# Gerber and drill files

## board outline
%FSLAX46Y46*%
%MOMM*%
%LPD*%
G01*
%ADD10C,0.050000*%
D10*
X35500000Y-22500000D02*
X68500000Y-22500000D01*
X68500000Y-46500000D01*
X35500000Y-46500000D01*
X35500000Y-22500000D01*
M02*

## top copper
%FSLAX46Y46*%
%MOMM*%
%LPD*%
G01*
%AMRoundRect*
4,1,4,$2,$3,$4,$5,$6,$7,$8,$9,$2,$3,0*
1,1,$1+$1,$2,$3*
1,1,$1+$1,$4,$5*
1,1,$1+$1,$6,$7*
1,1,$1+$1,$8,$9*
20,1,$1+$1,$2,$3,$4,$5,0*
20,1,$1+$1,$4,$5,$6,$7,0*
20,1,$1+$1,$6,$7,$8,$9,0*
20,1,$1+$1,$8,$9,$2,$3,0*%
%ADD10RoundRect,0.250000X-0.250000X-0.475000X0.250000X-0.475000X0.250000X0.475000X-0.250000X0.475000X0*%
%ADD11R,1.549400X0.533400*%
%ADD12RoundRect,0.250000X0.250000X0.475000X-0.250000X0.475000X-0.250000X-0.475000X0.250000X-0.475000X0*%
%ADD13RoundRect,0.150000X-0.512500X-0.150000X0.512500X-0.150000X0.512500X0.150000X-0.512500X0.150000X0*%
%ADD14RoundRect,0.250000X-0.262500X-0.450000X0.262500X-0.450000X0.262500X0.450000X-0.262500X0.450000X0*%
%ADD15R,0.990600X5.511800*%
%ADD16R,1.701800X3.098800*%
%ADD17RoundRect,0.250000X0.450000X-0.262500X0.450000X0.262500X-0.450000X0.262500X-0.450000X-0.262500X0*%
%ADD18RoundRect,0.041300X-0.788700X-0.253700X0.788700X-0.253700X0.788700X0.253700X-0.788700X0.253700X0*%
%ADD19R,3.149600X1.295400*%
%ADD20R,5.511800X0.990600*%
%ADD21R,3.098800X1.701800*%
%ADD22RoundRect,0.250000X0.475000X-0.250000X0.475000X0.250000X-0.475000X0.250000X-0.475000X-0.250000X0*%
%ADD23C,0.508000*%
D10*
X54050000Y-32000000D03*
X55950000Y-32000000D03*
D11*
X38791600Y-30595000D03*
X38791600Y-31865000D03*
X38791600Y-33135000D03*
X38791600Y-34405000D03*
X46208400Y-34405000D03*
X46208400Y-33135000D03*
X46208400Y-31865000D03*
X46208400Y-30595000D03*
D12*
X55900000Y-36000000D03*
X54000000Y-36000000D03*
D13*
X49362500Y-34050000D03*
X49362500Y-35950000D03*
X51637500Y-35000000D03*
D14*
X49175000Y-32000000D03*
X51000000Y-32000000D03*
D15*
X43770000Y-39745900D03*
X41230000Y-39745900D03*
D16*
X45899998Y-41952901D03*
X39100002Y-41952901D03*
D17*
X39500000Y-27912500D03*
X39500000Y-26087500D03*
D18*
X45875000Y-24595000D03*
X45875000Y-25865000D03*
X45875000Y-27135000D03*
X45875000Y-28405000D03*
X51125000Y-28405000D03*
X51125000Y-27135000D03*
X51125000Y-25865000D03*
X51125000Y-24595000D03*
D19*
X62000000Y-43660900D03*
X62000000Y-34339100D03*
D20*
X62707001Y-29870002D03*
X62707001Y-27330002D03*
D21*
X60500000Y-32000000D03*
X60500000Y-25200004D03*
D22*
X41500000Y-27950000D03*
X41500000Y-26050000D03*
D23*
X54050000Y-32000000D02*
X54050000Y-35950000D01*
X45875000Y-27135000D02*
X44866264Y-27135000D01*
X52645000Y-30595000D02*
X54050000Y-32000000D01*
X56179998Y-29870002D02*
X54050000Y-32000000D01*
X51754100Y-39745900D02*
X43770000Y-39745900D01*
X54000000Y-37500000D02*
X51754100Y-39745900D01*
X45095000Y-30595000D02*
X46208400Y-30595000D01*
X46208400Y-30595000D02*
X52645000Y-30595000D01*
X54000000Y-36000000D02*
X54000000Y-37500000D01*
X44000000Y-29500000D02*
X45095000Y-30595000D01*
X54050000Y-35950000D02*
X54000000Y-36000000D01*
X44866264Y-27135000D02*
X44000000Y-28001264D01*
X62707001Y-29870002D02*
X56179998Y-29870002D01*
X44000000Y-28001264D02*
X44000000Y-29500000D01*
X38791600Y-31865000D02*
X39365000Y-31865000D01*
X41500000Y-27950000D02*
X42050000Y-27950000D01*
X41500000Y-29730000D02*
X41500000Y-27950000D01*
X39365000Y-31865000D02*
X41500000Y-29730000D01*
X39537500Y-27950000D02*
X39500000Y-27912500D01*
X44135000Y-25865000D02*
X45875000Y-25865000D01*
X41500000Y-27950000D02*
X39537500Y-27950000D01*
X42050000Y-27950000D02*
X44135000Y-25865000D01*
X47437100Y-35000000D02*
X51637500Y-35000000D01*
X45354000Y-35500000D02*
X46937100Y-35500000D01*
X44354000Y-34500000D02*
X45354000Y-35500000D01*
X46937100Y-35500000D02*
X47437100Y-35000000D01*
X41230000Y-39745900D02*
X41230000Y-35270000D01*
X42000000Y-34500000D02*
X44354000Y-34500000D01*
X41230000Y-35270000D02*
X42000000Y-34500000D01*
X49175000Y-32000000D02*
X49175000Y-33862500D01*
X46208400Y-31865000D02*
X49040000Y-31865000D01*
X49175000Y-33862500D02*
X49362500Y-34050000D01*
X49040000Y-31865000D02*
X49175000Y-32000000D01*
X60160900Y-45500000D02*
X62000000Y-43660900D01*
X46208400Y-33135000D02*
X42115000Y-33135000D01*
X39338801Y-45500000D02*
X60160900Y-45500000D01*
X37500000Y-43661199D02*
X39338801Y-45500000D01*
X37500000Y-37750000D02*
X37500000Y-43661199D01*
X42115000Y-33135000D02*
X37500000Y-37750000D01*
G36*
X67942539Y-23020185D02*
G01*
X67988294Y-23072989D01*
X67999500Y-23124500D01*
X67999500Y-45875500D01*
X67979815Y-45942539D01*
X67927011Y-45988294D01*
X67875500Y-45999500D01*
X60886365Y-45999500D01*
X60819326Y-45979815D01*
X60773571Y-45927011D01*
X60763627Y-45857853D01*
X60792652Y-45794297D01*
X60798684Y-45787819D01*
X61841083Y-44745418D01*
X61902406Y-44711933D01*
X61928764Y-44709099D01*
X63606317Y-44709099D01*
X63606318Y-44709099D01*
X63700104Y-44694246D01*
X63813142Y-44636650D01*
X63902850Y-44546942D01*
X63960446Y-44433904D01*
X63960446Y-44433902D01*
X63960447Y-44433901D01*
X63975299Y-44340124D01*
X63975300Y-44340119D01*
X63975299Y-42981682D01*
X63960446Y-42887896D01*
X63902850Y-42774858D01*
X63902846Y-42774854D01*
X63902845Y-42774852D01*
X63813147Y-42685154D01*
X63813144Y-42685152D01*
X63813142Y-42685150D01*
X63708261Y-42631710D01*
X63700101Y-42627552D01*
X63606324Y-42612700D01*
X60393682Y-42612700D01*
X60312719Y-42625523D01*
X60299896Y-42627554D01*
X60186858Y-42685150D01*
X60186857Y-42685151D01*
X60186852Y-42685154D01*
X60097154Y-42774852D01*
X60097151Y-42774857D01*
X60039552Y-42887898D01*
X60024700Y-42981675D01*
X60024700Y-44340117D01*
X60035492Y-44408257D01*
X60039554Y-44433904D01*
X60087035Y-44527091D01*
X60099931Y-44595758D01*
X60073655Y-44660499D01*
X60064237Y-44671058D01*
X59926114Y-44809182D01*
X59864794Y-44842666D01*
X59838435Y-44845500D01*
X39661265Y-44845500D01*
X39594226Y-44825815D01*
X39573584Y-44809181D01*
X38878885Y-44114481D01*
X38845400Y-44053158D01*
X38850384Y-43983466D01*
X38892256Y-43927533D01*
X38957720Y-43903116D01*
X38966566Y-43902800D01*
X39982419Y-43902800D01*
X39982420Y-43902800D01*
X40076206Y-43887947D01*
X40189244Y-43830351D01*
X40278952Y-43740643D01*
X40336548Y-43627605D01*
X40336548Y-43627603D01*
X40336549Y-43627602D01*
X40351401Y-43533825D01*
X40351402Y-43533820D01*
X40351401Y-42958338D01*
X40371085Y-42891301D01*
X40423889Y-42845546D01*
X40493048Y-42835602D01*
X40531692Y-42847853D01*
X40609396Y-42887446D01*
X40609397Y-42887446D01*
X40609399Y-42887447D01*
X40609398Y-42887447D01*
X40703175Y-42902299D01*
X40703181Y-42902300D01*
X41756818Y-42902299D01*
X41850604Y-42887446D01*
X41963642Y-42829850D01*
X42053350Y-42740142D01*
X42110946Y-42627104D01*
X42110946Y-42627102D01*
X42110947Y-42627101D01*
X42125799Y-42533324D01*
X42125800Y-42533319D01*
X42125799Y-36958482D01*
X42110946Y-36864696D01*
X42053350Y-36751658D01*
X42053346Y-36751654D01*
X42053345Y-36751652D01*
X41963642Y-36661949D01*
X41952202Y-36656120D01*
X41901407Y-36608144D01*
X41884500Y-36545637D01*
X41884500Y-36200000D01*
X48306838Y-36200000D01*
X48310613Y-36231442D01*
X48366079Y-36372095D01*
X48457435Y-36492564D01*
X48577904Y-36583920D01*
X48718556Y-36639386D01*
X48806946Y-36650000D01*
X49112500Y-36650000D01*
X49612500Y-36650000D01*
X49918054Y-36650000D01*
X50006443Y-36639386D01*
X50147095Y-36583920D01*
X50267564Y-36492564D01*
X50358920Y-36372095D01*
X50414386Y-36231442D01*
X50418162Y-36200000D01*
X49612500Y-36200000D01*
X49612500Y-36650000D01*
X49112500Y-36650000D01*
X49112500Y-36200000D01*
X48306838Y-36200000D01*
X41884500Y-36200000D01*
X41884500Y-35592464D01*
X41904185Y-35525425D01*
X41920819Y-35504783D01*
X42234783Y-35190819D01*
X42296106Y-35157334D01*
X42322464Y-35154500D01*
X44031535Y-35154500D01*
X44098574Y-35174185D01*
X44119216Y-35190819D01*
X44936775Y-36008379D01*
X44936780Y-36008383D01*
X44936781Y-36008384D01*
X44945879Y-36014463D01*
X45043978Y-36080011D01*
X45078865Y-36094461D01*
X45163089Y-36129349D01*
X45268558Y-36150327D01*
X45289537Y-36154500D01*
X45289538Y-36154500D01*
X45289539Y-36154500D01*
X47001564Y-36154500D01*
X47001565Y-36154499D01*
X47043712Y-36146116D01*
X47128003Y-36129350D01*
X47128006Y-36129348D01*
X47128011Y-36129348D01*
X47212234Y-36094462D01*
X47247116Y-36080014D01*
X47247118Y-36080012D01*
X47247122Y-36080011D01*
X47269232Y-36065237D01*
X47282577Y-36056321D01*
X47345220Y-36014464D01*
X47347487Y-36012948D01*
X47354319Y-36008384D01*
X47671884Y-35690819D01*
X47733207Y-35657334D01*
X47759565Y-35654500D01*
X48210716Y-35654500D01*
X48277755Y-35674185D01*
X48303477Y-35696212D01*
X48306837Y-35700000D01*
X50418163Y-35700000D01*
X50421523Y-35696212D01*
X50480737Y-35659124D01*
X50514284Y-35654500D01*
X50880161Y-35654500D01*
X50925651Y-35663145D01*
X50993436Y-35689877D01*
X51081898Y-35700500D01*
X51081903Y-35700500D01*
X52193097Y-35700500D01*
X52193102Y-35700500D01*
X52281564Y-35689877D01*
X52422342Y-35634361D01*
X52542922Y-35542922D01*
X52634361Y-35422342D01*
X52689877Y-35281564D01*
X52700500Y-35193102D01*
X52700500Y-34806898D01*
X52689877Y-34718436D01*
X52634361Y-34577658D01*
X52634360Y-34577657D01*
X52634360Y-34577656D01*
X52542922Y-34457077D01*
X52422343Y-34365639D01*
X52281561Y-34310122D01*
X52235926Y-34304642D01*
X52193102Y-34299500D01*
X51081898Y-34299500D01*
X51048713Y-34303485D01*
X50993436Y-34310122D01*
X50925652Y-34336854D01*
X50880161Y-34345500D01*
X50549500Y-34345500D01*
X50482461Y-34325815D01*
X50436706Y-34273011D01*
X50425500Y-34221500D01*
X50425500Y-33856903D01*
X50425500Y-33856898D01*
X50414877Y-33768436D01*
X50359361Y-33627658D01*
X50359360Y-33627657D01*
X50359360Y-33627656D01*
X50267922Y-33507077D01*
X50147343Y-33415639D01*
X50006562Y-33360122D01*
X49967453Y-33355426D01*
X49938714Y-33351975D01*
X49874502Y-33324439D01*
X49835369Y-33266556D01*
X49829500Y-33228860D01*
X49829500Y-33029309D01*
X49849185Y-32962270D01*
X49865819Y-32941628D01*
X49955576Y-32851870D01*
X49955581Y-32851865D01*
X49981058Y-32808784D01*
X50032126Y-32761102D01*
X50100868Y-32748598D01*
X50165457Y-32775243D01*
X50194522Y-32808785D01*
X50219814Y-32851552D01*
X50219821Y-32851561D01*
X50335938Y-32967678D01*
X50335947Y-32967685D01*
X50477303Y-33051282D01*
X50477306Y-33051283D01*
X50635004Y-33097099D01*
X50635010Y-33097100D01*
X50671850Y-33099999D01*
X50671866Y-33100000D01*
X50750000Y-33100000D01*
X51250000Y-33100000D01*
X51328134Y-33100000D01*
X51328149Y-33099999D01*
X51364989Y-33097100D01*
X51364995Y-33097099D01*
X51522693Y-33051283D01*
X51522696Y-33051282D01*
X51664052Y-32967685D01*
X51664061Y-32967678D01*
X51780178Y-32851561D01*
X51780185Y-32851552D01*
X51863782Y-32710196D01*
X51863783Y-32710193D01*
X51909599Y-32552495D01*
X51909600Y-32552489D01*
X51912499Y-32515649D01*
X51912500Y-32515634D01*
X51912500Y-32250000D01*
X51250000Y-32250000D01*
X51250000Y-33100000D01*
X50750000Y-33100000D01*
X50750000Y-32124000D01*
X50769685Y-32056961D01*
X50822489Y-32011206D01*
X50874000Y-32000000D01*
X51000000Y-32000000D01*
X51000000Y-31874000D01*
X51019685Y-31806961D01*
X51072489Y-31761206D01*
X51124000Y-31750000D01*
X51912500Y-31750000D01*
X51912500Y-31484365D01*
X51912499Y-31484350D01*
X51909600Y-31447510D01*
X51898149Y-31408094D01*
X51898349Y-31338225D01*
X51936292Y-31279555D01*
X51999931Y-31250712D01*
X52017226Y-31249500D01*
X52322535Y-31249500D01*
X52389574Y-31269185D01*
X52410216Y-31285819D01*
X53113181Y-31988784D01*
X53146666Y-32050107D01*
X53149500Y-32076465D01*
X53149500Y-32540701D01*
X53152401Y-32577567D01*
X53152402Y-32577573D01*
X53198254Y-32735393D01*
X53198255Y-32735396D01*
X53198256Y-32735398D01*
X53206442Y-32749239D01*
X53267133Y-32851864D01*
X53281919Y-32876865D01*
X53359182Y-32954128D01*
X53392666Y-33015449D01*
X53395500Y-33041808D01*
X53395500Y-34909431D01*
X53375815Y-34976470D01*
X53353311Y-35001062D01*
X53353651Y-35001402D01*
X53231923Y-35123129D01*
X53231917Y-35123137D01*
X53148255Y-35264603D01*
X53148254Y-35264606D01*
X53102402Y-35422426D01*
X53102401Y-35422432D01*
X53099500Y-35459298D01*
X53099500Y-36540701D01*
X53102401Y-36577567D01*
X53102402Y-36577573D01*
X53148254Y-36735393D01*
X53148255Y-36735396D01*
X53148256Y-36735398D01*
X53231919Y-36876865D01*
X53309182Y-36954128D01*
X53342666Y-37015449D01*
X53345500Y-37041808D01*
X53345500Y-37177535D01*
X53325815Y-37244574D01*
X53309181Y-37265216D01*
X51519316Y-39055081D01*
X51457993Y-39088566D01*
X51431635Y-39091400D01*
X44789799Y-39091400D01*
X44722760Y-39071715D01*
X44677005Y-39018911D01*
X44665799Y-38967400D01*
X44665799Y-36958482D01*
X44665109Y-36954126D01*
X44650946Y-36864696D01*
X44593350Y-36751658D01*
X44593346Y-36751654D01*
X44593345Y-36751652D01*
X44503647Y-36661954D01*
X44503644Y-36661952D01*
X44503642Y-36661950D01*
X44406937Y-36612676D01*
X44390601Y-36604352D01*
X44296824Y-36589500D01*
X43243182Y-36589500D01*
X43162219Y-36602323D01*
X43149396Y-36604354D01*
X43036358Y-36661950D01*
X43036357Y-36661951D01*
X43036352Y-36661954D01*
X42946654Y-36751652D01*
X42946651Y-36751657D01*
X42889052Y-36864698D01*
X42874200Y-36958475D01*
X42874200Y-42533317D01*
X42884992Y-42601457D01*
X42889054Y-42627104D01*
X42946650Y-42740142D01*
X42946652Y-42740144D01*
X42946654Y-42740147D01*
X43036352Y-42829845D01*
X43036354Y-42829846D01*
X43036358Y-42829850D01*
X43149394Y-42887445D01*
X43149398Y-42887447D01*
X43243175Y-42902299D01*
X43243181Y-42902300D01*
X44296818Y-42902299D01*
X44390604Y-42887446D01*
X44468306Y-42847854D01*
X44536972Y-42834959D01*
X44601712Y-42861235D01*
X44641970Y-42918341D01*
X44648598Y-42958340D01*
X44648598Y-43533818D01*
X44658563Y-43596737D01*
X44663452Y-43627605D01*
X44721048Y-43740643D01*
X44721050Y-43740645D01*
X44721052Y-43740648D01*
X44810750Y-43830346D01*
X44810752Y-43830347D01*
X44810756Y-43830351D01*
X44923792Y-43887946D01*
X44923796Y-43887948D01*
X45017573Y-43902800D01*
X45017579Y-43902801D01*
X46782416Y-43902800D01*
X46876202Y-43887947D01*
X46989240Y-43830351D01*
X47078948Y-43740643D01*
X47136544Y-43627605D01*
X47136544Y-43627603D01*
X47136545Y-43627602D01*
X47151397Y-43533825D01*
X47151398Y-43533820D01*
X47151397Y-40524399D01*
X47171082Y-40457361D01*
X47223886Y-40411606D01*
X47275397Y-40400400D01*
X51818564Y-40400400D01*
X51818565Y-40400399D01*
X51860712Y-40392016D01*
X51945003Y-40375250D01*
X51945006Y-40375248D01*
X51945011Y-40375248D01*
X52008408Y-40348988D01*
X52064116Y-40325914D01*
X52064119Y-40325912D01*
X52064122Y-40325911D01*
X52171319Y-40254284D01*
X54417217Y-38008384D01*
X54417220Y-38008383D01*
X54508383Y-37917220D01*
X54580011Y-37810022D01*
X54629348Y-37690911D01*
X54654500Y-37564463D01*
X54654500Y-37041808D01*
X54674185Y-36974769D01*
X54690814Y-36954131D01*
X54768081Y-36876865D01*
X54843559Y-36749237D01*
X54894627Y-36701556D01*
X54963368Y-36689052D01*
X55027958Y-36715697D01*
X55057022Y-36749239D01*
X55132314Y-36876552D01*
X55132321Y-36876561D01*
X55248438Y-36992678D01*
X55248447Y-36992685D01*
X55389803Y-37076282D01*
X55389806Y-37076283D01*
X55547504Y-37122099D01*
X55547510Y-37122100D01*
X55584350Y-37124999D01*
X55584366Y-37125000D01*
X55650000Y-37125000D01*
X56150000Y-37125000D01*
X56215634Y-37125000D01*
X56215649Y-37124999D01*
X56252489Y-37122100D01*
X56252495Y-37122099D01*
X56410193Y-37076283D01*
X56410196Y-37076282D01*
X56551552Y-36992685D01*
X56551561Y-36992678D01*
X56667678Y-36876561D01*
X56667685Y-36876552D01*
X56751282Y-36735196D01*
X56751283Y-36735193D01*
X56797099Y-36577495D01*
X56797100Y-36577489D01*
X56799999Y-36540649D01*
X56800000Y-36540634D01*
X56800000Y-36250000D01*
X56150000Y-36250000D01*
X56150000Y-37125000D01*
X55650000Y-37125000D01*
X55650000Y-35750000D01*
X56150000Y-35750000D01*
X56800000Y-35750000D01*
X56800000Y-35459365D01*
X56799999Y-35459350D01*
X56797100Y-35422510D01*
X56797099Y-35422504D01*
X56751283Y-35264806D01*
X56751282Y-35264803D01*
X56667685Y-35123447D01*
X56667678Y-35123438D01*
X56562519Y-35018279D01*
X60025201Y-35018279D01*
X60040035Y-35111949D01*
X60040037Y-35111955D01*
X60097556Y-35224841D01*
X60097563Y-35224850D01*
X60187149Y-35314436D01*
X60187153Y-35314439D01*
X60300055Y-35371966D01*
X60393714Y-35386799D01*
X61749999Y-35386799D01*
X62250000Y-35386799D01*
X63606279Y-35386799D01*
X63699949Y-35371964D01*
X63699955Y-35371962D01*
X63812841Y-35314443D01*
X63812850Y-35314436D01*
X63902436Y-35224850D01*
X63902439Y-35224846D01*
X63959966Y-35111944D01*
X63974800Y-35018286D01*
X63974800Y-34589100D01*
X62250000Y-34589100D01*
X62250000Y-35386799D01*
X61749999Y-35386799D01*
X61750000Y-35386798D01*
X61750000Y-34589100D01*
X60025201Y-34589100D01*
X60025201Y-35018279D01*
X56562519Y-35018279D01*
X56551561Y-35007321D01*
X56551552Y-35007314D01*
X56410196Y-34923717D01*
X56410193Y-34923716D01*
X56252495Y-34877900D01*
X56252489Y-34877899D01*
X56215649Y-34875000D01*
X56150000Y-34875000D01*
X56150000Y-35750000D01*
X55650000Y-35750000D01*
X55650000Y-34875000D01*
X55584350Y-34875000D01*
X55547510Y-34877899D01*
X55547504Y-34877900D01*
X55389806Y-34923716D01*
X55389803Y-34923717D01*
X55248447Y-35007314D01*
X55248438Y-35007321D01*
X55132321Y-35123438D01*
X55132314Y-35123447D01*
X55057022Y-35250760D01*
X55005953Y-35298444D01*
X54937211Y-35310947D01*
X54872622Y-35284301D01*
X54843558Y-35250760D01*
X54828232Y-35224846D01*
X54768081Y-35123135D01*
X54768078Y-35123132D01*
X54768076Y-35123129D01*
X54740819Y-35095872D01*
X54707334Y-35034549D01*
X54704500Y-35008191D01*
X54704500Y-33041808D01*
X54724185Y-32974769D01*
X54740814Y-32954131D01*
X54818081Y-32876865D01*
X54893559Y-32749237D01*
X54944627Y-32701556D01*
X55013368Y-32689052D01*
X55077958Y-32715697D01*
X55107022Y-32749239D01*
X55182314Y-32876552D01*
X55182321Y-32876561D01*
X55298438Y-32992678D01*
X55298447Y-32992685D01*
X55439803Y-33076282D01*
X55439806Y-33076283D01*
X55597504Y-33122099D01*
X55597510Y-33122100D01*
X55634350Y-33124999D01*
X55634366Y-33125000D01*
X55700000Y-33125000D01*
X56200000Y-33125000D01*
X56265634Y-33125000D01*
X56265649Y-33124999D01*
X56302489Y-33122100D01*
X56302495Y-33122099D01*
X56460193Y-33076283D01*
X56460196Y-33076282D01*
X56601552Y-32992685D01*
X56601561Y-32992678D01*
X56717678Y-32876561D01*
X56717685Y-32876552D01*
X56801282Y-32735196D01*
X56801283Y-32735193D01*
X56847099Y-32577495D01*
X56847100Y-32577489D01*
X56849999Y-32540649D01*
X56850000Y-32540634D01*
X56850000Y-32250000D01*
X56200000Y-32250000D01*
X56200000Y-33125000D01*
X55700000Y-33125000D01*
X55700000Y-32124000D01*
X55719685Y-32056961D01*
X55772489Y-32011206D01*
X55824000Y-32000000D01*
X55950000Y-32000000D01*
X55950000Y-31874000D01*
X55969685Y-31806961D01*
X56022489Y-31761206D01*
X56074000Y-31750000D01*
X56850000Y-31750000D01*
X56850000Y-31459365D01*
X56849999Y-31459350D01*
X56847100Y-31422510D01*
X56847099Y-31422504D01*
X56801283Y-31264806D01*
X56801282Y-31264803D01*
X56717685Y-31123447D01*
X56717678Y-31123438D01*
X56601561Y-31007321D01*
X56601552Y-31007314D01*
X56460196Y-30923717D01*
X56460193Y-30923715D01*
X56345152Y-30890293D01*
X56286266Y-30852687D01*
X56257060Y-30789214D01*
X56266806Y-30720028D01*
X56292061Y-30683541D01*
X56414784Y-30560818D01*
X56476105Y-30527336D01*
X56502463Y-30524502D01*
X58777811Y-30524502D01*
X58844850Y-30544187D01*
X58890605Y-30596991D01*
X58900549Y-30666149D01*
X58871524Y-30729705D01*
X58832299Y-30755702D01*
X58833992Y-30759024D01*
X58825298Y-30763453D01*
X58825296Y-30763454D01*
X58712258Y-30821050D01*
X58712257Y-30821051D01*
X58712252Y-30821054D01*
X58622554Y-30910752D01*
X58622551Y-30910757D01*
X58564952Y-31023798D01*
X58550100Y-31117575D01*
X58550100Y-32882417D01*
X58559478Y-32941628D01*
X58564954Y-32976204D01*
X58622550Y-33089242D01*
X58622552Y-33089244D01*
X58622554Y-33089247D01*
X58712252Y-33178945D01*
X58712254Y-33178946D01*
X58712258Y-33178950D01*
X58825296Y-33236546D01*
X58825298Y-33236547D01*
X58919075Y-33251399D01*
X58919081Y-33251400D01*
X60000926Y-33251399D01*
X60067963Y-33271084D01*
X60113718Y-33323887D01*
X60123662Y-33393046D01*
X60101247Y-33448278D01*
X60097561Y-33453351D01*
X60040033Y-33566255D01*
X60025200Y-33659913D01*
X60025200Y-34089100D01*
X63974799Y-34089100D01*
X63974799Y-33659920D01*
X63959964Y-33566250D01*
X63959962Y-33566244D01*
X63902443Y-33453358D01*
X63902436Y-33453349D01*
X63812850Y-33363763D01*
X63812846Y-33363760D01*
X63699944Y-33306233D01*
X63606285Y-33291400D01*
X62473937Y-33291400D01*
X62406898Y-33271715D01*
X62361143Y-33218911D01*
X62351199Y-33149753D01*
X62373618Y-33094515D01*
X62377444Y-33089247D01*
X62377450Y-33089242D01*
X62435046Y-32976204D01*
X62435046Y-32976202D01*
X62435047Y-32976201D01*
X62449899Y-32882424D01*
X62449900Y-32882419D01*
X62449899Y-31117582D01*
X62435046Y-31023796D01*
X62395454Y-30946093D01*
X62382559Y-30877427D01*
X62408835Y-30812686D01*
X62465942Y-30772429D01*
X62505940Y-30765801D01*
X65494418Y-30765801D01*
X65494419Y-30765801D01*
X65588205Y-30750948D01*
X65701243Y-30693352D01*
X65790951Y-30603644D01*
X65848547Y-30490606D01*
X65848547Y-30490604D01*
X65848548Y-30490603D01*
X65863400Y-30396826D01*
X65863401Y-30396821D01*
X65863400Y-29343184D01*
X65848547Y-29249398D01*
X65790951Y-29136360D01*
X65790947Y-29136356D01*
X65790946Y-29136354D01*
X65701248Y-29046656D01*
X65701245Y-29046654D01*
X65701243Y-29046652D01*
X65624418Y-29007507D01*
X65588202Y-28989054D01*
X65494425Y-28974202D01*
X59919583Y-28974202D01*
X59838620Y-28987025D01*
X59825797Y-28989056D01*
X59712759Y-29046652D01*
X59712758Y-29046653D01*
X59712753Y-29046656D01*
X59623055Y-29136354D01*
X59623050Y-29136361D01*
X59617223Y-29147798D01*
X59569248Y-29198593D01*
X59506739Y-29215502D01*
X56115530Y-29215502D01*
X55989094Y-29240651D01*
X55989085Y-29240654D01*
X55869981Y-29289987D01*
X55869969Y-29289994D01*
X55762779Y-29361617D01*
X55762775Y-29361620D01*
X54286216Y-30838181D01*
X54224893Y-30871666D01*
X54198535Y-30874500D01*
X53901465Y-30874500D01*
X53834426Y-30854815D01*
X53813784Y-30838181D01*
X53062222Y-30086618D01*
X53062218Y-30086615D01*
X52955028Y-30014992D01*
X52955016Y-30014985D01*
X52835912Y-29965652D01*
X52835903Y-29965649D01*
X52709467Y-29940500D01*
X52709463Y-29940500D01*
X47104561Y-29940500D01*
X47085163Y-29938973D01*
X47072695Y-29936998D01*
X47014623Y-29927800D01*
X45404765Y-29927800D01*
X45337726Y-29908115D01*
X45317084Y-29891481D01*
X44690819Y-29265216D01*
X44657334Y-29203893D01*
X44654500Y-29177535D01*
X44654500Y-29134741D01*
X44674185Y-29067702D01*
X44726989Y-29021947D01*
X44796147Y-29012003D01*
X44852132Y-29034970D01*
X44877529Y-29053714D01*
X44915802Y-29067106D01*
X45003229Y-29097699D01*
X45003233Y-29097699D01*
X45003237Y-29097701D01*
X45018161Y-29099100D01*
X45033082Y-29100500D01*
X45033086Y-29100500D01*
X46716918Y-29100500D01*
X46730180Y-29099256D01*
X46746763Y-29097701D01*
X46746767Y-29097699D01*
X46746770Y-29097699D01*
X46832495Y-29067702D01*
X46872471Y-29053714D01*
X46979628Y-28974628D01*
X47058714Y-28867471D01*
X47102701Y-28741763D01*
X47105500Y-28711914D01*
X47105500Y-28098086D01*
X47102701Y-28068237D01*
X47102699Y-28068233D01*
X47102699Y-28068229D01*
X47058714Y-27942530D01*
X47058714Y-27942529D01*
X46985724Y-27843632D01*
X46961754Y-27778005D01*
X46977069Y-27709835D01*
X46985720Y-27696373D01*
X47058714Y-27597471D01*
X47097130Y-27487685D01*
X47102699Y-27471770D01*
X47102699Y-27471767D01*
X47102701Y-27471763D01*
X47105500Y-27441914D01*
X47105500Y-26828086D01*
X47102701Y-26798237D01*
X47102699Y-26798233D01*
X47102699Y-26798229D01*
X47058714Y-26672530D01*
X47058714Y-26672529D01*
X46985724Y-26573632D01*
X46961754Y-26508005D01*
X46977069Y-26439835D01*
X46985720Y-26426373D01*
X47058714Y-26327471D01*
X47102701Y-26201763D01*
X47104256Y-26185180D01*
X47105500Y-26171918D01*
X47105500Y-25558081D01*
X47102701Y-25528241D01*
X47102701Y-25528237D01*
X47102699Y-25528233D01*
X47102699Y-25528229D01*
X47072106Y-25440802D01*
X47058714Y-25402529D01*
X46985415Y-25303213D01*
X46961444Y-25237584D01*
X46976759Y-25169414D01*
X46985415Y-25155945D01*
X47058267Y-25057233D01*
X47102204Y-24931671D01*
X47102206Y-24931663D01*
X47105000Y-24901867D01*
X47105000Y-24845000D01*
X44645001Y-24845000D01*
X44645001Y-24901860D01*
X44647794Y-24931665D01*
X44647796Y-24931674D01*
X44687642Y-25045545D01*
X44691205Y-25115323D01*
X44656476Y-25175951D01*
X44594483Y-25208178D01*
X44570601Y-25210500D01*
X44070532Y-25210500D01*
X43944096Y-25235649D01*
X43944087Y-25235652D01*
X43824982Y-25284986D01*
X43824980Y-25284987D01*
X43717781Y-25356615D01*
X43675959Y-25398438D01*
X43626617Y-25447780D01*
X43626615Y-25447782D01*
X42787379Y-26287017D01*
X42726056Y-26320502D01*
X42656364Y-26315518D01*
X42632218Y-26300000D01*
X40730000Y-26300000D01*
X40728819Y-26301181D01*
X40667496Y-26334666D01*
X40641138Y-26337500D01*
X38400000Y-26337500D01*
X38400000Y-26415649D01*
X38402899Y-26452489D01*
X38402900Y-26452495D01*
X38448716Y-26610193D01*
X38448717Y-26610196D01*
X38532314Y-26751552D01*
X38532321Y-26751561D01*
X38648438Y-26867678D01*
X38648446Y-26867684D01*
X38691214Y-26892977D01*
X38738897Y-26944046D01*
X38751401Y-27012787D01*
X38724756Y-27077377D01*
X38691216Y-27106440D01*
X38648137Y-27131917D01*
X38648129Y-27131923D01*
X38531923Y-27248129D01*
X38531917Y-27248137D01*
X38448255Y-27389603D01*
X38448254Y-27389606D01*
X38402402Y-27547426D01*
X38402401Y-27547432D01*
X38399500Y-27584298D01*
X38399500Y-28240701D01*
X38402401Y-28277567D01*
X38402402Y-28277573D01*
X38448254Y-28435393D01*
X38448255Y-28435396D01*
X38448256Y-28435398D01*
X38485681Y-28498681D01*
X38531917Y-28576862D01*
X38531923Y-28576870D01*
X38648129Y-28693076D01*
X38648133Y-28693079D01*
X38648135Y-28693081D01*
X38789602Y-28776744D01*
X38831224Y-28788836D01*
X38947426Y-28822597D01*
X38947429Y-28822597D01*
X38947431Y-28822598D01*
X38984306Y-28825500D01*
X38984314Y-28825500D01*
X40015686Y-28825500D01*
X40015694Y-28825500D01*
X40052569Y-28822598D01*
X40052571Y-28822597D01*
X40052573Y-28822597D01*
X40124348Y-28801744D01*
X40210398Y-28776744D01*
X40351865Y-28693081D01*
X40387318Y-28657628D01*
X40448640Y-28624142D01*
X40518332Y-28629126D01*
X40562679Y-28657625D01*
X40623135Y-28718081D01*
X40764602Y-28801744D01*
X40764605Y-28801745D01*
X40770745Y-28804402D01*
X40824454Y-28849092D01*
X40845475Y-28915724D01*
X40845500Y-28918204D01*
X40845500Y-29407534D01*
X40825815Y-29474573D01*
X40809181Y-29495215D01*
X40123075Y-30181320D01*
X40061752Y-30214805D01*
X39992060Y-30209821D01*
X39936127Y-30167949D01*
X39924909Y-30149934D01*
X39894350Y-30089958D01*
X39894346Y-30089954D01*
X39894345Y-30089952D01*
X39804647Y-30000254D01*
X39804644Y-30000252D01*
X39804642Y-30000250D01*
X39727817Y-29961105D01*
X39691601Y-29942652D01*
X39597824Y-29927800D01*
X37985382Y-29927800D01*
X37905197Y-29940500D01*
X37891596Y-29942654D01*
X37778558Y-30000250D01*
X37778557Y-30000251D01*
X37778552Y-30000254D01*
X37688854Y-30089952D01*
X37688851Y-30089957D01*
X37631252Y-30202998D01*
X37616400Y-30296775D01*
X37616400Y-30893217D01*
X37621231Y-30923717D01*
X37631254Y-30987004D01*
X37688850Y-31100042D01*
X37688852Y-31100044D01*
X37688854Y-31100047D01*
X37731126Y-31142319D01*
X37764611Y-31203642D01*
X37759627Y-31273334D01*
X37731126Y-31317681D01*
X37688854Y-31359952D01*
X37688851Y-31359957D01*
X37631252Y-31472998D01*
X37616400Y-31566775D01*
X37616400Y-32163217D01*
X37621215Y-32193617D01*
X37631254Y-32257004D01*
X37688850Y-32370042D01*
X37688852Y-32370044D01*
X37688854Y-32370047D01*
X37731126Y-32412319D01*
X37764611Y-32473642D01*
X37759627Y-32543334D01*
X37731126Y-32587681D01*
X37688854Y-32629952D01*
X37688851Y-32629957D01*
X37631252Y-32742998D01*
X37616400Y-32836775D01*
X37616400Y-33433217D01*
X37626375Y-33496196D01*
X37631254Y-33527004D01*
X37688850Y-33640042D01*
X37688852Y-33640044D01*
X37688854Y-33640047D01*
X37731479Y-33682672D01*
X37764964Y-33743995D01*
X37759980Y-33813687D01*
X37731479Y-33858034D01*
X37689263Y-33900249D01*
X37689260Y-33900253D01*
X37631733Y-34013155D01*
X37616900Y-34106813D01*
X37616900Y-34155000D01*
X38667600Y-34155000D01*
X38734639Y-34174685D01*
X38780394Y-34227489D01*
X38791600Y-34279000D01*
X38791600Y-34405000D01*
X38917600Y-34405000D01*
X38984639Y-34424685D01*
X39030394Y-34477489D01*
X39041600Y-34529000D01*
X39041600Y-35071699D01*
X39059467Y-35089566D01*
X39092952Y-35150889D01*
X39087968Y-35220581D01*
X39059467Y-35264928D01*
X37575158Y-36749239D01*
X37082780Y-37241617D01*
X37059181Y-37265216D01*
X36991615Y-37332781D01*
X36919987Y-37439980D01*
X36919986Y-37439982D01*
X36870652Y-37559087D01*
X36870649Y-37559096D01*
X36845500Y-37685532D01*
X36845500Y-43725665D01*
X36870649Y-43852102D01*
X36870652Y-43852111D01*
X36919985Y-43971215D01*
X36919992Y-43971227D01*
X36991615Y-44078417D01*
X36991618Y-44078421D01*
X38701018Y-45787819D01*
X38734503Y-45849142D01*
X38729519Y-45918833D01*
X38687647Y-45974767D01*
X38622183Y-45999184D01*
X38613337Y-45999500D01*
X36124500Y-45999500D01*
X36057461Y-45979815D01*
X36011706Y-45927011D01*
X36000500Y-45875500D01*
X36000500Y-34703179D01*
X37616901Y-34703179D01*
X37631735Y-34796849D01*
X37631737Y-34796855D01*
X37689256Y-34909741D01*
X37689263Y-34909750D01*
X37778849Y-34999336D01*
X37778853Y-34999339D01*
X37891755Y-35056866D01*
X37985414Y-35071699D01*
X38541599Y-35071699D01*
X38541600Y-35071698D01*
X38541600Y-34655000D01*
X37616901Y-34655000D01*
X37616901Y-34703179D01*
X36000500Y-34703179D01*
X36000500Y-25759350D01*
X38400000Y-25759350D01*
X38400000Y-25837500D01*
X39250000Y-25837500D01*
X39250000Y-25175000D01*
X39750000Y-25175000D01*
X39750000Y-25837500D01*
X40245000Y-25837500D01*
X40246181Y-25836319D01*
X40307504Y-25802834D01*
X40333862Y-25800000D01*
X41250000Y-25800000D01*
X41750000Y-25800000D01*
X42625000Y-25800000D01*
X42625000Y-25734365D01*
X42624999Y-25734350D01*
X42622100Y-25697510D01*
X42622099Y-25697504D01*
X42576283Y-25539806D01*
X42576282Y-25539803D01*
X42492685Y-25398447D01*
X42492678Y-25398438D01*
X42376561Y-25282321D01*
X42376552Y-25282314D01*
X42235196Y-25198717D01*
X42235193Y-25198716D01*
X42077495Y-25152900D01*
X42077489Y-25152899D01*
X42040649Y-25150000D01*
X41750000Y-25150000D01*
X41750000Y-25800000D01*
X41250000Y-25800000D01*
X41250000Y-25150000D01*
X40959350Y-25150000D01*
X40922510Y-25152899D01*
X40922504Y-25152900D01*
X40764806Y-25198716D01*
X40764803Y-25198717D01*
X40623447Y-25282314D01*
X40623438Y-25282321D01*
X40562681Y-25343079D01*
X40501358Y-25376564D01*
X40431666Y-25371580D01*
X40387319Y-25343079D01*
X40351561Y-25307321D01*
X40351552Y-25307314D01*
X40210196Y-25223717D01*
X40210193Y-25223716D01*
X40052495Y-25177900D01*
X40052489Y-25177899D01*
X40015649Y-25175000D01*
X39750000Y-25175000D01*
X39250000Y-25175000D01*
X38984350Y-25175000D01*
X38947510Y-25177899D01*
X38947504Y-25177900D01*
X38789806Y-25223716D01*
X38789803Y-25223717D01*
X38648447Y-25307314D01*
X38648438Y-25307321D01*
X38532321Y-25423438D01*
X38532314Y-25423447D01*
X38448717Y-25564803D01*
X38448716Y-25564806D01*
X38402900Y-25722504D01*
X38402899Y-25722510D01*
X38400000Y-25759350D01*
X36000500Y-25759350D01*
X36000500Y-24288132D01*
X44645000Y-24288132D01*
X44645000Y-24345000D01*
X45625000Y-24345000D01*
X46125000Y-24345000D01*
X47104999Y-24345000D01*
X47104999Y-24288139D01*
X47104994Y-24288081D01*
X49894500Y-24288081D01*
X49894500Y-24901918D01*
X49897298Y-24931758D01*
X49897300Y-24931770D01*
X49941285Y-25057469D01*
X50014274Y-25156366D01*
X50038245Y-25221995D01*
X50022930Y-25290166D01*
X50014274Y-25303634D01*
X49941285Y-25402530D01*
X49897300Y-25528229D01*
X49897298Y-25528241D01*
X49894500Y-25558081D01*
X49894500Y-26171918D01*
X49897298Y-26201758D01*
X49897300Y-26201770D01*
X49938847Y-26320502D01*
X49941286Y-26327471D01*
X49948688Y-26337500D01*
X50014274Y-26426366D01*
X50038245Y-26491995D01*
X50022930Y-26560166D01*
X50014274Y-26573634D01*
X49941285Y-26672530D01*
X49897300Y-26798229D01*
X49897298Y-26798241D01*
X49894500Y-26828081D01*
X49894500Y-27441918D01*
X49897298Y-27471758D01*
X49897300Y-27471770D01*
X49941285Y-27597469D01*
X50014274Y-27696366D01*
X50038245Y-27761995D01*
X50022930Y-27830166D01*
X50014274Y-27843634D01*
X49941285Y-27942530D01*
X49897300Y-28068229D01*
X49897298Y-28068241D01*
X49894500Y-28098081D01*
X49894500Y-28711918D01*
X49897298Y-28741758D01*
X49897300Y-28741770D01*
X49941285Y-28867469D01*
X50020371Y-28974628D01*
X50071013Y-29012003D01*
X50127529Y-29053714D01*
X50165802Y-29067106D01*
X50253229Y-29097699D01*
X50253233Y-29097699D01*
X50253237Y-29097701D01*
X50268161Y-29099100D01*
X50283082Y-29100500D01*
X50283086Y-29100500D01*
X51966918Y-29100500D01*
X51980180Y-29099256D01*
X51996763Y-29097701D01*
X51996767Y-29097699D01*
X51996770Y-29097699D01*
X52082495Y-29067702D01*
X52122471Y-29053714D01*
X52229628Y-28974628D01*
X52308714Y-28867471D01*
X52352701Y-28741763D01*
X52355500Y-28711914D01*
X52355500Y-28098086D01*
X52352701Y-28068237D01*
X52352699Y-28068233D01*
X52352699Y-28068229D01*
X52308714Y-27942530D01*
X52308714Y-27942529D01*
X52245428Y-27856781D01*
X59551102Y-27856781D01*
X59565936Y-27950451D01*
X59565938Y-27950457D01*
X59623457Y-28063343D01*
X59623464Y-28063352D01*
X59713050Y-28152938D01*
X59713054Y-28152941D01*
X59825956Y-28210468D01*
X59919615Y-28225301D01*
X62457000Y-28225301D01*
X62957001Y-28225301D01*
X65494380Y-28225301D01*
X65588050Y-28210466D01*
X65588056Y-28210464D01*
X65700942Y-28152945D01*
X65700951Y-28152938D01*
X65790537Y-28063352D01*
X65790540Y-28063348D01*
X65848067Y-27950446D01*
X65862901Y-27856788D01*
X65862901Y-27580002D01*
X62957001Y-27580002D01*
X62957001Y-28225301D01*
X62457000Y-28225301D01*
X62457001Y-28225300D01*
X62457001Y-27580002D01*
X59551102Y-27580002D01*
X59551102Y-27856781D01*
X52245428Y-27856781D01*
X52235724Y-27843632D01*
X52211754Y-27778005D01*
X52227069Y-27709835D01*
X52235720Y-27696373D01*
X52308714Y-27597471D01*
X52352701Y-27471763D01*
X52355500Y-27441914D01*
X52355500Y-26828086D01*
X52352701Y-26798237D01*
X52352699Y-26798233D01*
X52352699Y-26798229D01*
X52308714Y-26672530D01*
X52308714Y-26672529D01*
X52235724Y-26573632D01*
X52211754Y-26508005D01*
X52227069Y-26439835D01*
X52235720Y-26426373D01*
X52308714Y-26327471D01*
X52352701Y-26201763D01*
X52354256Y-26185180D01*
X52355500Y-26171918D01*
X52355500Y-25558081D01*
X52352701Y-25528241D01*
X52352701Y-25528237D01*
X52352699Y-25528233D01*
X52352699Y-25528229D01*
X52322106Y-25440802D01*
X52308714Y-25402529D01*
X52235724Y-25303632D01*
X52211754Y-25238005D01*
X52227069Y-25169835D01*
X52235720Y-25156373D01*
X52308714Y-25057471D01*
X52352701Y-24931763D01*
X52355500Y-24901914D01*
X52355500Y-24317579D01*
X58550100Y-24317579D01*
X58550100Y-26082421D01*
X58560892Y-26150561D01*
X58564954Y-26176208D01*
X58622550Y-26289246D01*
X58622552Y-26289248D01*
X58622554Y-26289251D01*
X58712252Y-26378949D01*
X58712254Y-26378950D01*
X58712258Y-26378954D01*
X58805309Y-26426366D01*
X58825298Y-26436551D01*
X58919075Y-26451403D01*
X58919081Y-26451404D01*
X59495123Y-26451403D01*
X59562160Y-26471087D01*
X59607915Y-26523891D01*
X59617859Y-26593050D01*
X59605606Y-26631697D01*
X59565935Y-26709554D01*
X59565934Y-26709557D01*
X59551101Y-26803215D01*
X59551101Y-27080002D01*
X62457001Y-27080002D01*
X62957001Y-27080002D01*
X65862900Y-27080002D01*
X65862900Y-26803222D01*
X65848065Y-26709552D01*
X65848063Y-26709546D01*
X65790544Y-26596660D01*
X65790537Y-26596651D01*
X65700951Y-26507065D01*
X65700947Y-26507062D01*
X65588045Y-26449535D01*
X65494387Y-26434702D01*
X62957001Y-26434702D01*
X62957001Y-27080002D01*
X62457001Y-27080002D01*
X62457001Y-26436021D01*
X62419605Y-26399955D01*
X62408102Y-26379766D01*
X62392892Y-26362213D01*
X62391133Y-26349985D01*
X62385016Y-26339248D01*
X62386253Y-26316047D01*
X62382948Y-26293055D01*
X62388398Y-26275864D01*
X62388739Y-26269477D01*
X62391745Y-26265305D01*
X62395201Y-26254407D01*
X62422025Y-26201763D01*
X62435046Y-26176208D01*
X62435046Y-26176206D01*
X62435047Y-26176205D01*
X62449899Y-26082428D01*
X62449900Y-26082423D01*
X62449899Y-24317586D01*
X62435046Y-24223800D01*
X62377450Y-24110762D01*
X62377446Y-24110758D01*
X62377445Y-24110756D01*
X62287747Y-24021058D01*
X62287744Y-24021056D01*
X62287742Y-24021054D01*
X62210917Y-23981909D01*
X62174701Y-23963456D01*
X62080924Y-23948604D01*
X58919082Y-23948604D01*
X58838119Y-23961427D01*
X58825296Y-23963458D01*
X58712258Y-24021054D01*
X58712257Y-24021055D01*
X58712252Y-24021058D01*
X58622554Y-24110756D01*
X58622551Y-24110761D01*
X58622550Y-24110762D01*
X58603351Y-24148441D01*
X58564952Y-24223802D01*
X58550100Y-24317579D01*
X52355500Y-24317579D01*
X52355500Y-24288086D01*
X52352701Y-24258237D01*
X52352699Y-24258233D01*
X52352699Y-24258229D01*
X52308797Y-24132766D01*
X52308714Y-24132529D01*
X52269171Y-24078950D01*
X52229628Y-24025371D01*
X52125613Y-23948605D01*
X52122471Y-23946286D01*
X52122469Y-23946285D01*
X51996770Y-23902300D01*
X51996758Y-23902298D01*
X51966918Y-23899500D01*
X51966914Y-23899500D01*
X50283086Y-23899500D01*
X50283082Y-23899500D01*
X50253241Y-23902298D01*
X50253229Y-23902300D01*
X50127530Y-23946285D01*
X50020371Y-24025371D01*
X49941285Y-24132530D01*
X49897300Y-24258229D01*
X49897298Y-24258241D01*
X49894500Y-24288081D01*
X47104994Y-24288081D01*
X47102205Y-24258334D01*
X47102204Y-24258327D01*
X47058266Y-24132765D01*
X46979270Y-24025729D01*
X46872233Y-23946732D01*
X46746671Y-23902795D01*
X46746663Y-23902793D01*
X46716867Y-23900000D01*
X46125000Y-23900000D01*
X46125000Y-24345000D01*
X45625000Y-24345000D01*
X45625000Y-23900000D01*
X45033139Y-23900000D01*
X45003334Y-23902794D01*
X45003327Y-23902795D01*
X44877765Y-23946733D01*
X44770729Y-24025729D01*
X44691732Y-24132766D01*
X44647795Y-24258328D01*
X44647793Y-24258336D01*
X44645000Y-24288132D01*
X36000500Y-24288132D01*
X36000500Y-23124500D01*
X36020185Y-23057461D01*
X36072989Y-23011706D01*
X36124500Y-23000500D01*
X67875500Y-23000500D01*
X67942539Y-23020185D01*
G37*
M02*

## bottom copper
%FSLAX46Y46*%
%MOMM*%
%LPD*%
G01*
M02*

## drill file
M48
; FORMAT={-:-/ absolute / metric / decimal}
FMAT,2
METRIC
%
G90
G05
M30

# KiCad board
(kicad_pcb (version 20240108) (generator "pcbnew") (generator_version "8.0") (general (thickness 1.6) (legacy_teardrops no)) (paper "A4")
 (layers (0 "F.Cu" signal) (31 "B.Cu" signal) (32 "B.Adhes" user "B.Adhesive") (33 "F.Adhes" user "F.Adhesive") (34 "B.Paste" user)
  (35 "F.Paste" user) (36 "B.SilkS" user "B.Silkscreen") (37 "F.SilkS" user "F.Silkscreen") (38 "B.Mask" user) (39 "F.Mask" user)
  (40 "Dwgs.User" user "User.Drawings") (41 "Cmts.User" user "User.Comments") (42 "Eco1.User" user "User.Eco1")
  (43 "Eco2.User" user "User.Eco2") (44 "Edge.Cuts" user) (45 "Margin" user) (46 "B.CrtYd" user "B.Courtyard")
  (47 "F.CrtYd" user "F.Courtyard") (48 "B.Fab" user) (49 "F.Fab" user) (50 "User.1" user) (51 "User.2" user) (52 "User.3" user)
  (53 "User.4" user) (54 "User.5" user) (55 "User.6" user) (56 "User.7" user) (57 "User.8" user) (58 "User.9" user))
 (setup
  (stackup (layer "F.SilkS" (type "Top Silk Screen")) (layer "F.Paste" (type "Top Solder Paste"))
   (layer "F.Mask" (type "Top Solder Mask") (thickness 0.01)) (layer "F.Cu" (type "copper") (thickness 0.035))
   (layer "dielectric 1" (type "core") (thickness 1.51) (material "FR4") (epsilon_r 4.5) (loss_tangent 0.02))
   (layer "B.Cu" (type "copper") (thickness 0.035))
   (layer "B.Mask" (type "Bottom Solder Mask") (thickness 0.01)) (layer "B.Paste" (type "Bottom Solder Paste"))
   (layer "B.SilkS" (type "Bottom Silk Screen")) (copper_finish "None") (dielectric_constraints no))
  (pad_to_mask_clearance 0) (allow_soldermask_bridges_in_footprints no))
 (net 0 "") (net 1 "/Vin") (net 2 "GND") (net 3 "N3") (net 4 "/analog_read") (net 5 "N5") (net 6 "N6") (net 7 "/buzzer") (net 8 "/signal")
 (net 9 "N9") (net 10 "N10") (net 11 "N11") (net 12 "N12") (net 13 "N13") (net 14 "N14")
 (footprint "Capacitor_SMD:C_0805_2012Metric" (layer "F.Cu") (at 55 32)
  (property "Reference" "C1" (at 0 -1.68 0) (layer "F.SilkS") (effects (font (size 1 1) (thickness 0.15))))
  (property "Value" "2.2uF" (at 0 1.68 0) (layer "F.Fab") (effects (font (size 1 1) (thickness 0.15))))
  (pad "1" smd roundrect (at -0.95 0) (size 1 1.45) (layers "F.Cu" "F.Paste" "F.Mask") (roundrect_rratio 0.25) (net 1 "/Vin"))
  (pad "2" smd roundrect (at 0.95 0) (size 1 1.45) (layers "F.Cu" "F.Paste" "F.Mask") (roundrect_rratio 0.25) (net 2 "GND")))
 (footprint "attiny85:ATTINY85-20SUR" (layer "F.Cu") (at 42.5 32.5)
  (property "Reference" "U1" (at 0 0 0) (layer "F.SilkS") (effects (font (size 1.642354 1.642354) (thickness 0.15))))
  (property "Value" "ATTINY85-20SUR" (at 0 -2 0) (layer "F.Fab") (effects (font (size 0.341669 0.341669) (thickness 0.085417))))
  (pad "1" smd rect (at -3.7084 -1.905) (size 1.5494 0.5334) (layers "F.Cu" "F.Paste" "F.Mask") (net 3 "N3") (solder_mask_margin 0.102))
  (pad "2" smd rect (at -3.7084 -0.635) (size 1.5494 0.5334) (layers "F.Cu" "F.Paste" "F.Mask") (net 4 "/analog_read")
   (solder_mask_margin 0.102))
  (pad "3" smd rect (at -3.7084 0.635) (size 1.5494 0.5334) (layers "F.Cu" "F.Paste" "F.Mask") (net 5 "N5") (solder_mask_margin 0.102))
  (pad "4" smd rect (at -3.7084 1.905) (size 1.5494 0.5334) (layers "F.Cu" "F.Paste" "F.Mask") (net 2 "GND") (solder_mask_margin 0.102))
  (pad "5" smd rect (at 3.7084 1.905) (size 1.5494 0.5334) (layers "F.Cu" "F.Paste" "F.Mask") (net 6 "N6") (solder_mask_margin 0.102))
  (pad "6" smd rect (at 3.7084 0.635) (size 1.5494 0.5334) (layers "F.Cu" "F.Paste" "F.Mask") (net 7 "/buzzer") (solder_mask_margin 0.102))
  (pad "7" smd rect (at 3.7084 -0.635) (size 1.5494 0.5334) (layers "F.Cu" "F.Paste" "F.Mask") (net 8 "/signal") (solder_mask_margin 0.102))
  (pad "8" smd rect (at 3.7084 -1.905) (size 1.5494 0.5334) (layers "F.Cu" "F.Paste" "F.Mask") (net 1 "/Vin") (solder_mask_margin 0.102)))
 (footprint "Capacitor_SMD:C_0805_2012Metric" (layer "F.Cu") (at 54.95 36 180)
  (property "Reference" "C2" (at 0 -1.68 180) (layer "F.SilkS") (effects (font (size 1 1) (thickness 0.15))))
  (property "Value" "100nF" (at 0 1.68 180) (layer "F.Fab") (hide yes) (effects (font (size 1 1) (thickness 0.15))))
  (pad "1" smd roundrect (at -0.95 0 180) (size 1 1.45) (layers "F.Cu" "F.Paste" "F.Mask") (roundrect_rratio 0.25) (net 2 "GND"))
  (pad "2" smd roundrect (at 0.95 0 180) (size 1 1.45) (layers "F.Cu" "F.Paste" "F.Mask") (roundrect_rratio 0.25) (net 1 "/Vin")))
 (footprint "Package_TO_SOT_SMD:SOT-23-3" (layer "F.Cu") (at 50.5 35)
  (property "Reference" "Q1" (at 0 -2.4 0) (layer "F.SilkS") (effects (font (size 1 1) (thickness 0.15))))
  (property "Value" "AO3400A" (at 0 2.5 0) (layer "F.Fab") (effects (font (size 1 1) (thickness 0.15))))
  (pad "1" smd roundrect (at -1.1375 -0.95) (size 1.325 0.6) (layers "F.Cu" "F.Paste" "F.Mask") (roundrect_rratio 0.25) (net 8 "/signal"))
  (pad "2" smd roundrect (at -1.1375 0.95) (size 1.325 0.6) (layers "F.Cu" "F.Paste" "F.Mask") (roundrect_rratio 0.25) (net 2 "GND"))
  (pad "3" smd roundrect (at 1.1375 0) (size 1.325 0.6) (layers "F.Cu" "F.Paste" "F.Mask") (roundrect_rratio 0.25) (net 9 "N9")))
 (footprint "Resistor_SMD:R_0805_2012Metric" (layer "F.Cu") (at 50.0875 32)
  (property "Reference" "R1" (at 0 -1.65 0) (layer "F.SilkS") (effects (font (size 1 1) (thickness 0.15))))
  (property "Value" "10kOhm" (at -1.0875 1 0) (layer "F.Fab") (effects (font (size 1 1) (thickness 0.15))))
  (pad "1" smd roundrect (at -0.9125 0) (size 1.025 1.4) (layers "F.Cu" "F.Paste" "F.Mask") (roundrect_rratio 0.243902) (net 8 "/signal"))
  (pad "2" smd roundrect (at 0.9125 0) (size 1.025 1.4) (layers "F.Cu" "F.Paste" "F.Mask") (roundrect_rratio 0.243902) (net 2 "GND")))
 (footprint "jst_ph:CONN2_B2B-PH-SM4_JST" (layer "F.Cu") (at 42.5 42 180)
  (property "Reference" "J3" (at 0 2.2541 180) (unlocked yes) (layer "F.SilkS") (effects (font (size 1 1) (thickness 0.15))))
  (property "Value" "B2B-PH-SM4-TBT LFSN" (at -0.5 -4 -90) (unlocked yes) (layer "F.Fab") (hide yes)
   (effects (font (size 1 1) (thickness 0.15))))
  (pad "1" smd rect (at -1.27 2.2541 180) (size 0.9906 5.5118) (layers "F.Cu" "F.Paste" "F.Mask") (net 1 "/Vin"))
  (pad "2" smd rect (at 1.27 2.2541 180) (size 0.9906 5.5118) (layers "F.Cu" "F.Paste" "F.Mask") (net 9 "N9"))
  (pad "3" smd rect (at -3.399998 0.047099 180) (size 1.7018 3.0988) (layers "F.Cu" "F.Paste" "F.Mask"))
  (pad "4" smd rect (at 3.399998 0.047099 180) (size 1.7018 3.0988) (layers "F.Cu" "F.Paste" "F.Mask")))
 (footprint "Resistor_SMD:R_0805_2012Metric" (layer "F.Cu") (at 39.5 27 90)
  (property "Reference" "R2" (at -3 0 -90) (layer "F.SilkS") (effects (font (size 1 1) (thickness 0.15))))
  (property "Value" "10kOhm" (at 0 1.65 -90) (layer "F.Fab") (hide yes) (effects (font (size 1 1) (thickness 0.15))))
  (pad "1" smd roundrect (at -0.9125 0 90) (size 1.025 1.4) (layers "F.Cu" "F.Paste" "F.Mask") (roundrect_rratio 0.243902)
   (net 4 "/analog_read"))
  (pad "2" smd roundrect (at 0.9125 0 90) (size 1.025 1.4) (layers "F.Cu" "F.Paste" "F.Mask") (roundrect_rratio 0.243902) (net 2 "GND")))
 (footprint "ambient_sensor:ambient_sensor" (layer "F.Cu") (at 48.5 26.5)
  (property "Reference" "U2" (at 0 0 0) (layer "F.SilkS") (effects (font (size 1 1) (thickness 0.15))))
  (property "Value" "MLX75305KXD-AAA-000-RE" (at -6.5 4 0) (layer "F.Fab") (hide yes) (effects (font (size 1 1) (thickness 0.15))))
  (pad "1" smd roundrect (at -2.625 -1.905) (size 1.66 0.59) (layers "F.Cu" "F.Paste" "F.Mask") (roundrect_rratio 0.07) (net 2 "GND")
   (solder_mask_margin 0.102))
  (pad "2" smd roundrect (at -2.625 -0.635) (size 1.66 0.59) (layers "F.Cu" "F.Paste" "F.Mask") (roundrect_rratio 0.07)
   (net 4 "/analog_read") (solder_mask_margin 0.102))
  (pad "3" smd roundrect (at -2.625 0.635) (size 1.66 0.59) (layers "F.Cu" "F.Paste" "F.Mask") (roundrect_rratio 0.07) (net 1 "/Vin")
   (solder_mask_margin 0.102))
  (pad "4" smd roundrect (at -2.625 1.905) (size 1.66 0.59) (layers "F.Cu" "F.Paste" "F.Mask") (roundrect_rratio 0.07) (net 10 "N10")
   (solder_mask_margin 0.102))
  (pad "5" smd roundrect (at 2.625 1.905) (size 1.66 0.59) (layers "F.Cu" "F.Paste" "F.Mask") (roundrect_rratio 0.07) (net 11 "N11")
   (solder_mask_margin 0.102))
  (pad "6" smd roundrect (at 2.625 0.635) (size 1.66 0.59) (layers "F.Cu" "F.Paste" "F.Mask") (roundrect_rratio 0.07) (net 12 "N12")
   (solder_mask_margin 0.102))
  (pad "7" smd roundrect (at 2.625 -0.635) (size 1.66 0.59) (layers "F.Cu" "F.Paste" "F.Mask") (roundrect_rratio 0.07) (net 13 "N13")
   (solder_mask_margin 0.102))
  (pad "8" smd roundrect (at 2.625 -1.905) (size 1.66 0.59) (layers "F.Cu" "F.Paste" "F.Mask") (roundrect_rratio 0.07) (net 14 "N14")
   (solder_mask_margin 0.102)))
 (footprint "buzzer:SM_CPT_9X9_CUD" (layer "F.Cu") (at 62 39 90)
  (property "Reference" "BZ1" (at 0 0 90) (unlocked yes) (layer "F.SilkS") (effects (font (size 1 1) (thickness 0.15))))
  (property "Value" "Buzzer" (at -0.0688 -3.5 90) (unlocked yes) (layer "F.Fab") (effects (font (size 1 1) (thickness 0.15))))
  (pad "1" smd rect (at -4.6609 0 90) (size 1.2954 3.1496) (layers "F.Cu" "F.Paste" "F.Mask") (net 7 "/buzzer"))
  (pad "2" smd rect (at 4.6609 0 90) (size 1.2954 3.1496) (layers "F.Cu" "F.Paste" "F.Mask") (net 2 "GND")))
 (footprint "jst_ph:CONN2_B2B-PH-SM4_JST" (layer "F.Cu") (at 60.452901 28.600002 90)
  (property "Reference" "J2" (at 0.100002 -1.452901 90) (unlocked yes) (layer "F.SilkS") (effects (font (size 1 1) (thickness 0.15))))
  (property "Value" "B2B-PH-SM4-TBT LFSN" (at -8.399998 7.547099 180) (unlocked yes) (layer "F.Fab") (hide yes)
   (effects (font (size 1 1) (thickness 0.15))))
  (pad "1" smd rect (at -1.27 2.2541 90) (size 0.9906 5.5118) (layers "F.Cu" "F.Paste" "F.Mask") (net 1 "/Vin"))
  (pad "2" smd rect (at 1.27 2.2541 90) (size 0.9906 5.5118) (layers "F.Cu" "F.Paste" "F.Mask") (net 2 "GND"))
  (pad "3" smd rect (at -3.399998 0.047099 90) (size 1.7018 3.0988) (layers "F.Cu" "F.Paste" "F.Mask"))
  (pad "4" smd rect (at 3.399998 0.047099 90) (size 1.7018 3.0988) (layers "F.Cu" "F.Paste" "F.Mask")))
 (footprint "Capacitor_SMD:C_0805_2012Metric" (layer "F.Cu") (at 41.5 27 90)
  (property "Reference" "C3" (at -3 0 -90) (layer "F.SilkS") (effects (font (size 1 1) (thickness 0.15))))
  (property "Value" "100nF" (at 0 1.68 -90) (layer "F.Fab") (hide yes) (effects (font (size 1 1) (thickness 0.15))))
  (pad "1" smd roundrect (at -0.95 0 90) (size 1 1.45) (layers "F.Cu" "F.Paste" "F.Mask") (roundrect_rratio 0.25) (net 4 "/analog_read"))
  (pad "2" smd roundrect (at 0.95 0 90) (size 1 1.45) (layers "F.Cu" "F.Paste" "F.Mask") (roundrect_rratio 0.25) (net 2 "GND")))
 (gr_rect (start 35.5 22.5) (end 68.5 46.5) (stroke (width 0.05) (type default)) (fill none) (layer "Edge.Cuts"))
 (segment (start 54.05 32) (end 54.05 35.95) (width 0.508) (layer "F.Cu") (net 1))
 (segment (start 45.875 27.135) (end 44.866264 27.135) (width 0.508) (layer "F.Cu") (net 1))
 (segment (start 52.645 30.595) (end 54.05 32) (width 0.508) (layer "F.Cu") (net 1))
 (segment (start 56.179998 29.870002) (end 54.05 32) (width 0.508) (layer "F.Cu") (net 1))
 (segment (start 51.7541 39.7459) (end 43.77 39.7459) (width 0.508) (layer "F.Cu") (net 1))
 (segment (start 54 37.5) (end 51.7541 39.7459) (width 0.508) (layer "F.Cu") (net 1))
 (segment (start 45.095 30.595) (end 46.2084 30.595) (width 0.508) (layer "F.Cu") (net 1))
 (segment (start 46.2084 30.595) (end 52.645 30.595) (width 0.508) (layer "F.Cu") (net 1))
 (segment (start 54 36) (end 54 37.5) (width 0.508) (layer "F.Cu") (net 1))
 (segment (start 44 29.5) (end 45.095 30.595) (width 0.508) (layer "F.Cu") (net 1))
 (segment (start 54.05 35.95) (end 54 36) (width 0.508) (layer "F.Cu") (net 1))
 (segment (start 44.866264 27.135) (end 44 28.001264) (width 0.508) (layer "F.Cu") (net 1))
 (segment (start 62.707001 29.870002) (end 56.179998 29.870002) (width 0.508) (layer "F.Cu") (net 1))
 (segment (start 44 28.001264) (end 44 29.5) (width 0.508) (layer "F.Cu") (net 1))
 (segment (start 38.7916 31.865) (end 39.365 31.865) (width 0.508) (layer "F.Cu") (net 4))
 (segment (start 41.5 27.95) (end 42.05 27.95) (width 0.508) (layer "F.Cu") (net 4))
 (segment (start 41.5 29.73) (end 41.5 27.95) (width 0.508) (layer "F.Cu") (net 4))
 (segment (start 39.365 31.865) (end 41.5 29.73) (width 0.508) (layer "F.Cu") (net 4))
 (segment (start 39.5375 27.95) (end 39.5 27.9125) (width 0.508) (layer "F.Cu") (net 4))
 (segment (start 44.135 25.865) (end 45.875 25.865) (width 0.508) (layer "F.Cu") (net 4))
 (segment (start 41.5 27.95) (end 39.5375 27.95) (width 0.508) (layer "F.Cu") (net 4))
 (segment (start 42.05 27.95) (end 44.135 25.865) (width 0.508) (layer "F.Cu") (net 4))
 (segment (start 47.4371 35) (end 51.6375 35) (width 0.508) (layer "F.Cu") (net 9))
 (segment (start 45.354 35.5) (end 46.9371 35.5) (width 0.508) (layer "F.Cu") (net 9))
 (segment (start 44.354 34.5) (end 45.354 35.5) (width 0.508) (layer "F.Cu") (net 9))
 (segment (start 46.9371 35.5) (end 47.4371 35) (width 0.508) (layer "F.Cu") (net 9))
 (segment (start 41.23 39.7459) (end 41.23 35.27) (width 0.508) (layer "F.Cu") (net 9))
 (segment (start 42 34.5) (end 44.354 34.5) (width 0.508) (layer "F.Cu") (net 9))
 (segment (start 41.23 35.27) (end 42 34.5) (width 0.508) (layer "F.Cu") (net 9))
 (segment (start 49.175 32) (end 49.175 33.8625) (width 0.508) (layer "F.Cu") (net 8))
 (segment (start 46.2084 31.865) (end 49.04 31.865) (width 0.508) (layer "F.Cu") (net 8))
 (segment (start 49.175 33.8625) (end 49.3625 34.05) (width 0.508) (layer "F.Cu") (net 8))
 (segment (start 49.04 31.865) (end 49.175 32) (width 0.508) (layer "F.Cu") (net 8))
 (segment (start 60.1609 45.5) (end 62 43.6609) (width 0.508) (layer "F.Cu") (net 7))
 (segment (start 46.2084 33.135) (end 42.115 33.135) (width 0.508) (layer "F.Cu") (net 7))
 (segment (start 39.338801 45.5) (end 60.1609 45.5) (width 0.508) (layer "F.Cu") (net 7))
 (segment (start 37.5 43.661199) (end 39.338801 45.5) (width 0.508) (layer "F.Cu") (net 7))
 (segment (start 37.5 37.75) (end 37.5 43.661199) (width 0.508) (layer "F.Cu") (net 7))
 (segment (start 42.115 33.135) (end 37.5 37.75) (width 0.508) (layer "F.Cu") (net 7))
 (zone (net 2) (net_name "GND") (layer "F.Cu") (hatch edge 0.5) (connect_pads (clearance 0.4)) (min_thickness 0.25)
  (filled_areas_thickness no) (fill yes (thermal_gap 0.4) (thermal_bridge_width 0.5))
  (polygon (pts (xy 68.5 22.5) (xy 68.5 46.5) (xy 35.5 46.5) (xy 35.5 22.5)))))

